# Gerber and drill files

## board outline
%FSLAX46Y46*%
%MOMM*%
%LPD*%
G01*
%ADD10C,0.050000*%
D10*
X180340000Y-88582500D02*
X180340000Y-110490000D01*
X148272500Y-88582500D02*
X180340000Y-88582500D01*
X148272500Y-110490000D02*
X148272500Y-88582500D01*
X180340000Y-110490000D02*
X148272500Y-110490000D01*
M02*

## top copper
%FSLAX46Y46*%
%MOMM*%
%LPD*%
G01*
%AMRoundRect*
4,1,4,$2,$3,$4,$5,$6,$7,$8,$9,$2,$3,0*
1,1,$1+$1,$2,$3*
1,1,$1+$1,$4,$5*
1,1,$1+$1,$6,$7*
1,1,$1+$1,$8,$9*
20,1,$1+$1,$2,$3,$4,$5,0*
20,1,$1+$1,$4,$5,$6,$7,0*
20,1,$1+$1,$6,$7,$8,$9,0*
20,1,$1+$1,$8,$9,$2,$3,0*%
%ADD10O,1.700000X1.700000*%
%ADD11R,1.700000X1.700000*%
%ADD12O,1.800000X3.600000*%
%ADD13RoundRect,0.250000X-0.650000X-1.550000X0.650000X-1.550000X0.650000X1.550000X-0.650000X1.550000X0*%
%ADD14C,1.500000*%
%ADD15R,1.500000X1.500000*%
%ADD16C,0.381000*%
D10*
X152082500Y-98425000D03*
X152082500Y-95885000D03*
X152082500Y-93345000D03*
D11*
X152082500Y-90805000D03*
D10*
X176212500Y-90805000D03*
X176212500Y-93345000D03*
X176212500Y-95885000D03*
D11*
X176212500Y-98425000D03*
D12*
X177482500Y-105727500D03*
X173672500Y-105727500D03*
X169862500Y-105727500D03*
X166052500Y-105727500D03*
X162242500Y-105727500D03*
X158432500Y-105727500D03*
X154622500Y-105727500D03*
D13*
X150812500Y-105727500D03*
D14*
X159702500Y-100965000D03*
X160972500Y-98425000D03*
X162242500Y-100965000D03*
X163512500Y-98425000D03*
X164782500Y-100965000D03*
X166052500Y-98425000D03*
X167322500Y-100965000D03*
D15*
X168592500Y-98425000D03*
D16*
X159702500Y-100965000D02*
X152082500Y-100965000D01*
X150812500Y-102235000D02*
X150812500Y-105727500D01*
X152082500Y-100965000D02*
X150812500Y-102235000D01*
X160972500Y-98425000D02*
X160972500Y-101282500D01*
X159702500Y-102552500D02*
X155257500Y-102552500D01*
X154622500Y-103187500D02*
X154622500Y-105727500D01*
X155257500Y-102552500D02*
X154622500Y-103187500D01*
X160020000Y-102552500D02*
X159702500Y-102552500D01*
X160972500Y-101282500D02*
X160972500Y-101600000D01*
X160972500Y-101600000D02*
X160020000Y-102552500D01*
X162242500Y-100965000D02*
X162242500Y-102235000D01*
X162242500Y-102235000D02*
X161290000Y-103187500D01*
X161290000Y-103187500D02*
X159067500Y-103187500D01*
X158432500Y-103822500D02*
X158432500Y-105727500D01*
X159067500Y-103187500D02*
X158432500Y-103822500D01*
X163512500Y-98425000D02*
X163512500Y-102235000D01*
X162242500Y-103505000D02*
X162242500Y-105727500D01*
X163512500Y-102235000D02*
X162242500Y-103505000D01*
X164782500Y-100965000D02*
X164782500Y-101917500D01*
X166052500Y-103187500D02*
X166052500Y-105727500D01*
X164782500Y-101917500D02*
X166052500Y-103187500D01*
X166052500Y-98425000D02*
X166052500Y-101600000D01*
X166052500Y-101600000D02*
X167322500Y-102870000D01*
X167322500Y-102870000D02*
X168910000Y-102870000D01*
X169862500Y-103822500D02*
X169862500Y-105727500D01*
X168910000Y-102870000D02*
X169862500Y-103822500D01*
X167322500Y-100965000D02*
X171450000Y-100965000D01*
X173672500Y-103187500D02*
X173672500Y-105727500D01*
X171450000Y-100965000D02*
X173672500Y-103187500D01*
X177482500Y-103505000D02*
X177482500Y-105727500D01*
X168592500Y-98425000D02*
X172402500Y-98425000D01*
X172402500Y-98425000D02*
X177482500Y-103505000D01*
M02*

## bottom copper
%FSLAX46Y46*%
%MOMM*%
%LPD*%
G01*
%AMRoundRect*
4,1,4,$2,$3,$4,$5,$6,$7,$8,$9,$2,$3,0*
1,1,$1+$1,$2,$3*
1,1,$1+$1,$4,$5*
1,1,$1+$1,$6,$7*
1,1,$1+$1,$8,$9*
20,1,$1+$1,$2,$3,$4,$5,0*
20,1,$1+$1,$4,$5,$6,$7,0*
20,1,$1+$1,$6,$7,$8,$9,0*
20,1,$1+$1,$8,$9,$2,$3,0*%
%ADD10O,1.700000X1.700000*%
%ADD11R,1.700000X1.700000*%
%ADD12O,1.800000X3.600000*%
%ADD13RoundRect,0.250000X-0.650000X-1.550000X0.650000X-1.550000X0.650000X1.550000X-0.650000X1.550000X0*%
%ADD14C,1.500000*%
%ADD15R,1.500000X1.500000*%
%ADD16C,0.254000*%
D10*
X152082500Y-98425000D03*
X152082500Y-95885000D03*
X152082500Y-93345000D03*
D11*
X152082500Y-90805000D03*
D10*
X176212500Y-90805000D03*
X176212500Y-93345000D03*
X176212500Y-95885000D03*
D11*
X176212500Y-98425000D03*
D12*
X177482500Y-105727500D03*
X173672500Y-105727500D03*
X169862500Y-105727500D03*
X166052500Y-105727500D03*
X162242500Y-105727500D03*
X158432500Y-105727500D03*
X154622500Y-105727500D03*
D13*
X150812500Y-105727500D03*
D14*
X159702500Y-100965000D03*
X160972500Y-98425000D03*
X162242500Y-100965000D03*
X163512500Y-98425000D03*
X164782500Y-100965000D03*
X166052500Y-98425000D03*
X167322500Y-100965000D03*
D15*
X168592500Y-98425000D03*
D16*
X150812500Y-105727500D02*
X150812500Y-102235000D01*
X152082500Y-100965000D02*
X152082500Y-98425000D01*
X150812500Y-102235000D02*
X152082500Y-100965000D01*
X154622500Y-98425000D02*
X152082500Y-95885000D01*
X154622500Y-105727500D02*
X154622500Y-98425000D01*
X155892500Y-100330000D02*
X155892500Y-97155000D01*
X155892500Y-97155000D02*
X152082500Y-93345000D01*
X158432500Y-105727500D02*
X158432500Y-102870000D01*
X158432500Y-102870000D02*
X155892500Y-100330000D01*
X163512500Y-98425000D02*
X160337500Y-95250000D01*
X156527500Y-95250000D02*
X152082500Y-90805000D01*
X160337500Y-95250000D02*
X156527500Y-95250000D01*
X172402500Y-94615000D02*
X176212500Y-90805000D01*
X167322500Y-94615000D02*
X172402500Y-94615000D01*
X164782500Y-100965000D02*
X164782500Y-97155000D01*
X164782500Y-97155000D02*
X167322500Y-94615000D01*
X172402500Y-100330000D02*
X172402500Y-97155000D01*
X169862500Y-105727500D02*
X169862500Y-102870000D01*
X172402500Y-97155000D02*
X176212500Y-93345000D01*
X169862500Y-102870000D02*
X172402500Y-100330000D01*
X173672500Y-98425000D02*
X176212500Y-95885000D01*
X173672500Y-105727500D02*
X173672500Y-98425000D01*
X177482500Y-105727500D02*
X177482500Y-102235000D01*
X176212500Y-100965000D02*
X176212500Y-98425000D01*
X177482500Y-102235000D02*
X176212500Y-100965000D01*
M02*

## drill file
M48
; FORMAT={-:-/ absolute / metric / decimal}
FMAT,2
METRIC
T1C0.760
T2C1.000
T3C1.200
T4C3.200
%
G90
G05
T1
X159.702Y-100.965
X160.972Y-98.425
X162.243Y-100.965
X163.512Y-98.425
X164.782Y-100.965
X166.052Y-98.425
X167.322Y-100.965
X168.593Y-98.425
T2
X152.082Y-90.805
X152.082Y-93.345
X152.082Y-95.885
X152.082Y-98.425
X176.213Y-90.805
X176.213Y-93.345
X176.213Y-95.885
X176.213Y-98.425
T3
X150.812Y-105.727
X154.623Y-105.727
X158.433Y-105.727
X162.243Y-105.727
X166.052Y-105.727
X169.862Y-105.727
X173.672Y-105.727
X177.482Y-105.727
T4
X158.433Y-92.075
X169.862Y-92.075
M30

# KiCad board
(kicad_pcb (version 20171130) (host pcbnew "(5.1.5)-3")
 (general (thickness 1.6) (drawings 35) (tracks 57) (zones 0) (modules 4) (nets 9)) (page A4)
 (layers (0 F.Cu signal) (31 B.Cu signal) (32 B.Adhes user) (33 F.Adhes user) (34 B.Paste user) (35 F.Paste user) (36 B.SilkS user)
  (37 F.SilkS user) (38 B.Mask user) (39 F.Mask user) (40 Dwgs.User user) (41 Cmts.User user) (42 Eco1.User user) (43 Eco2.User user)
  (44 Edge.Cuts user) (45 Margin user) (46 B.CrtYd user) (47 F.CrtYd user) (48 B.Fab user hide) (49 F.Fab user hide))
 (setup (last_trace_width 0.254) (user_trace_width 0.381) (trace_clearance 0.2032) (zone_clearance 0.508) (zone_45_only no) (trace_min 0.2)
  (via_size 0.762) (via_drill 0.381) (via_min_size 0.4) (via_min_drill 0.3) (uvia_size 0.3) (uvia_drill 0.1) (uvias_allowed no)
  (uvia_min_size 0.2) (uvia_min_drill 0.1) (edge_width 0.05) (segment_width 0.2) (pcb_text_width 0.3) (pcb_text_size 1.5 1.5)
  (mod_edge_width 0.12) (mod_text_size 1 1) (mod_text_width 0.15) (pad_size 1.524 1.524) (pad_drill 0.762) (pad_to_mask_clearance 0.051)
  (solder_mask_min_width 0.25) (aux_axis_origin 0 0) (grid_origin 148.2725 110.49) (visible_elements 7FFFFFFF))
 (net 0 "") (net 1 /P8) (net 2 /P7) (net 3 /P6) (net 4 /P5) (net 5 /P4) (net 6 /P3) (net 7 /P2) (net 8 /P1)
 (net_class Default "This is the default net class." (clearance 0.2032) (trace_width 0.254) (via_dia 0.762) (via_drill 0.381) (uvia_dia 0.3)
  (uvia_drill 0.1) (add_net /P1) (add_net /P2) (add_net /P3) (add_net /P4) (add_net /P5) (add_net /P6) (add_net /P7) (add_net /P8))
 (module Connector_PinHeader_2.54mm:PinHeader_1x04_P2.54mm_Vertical (layer F.Cu) (at 152.0825 90.805)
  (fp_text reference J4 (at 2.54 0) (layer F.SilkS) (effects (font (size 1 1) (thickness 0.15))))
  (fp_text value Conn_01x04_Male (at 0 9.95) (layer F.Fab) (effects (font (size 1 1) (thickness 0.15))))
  (pad 4 thru_hole oval (at 0 7.62) (size 1.7 1.7) (drill 1) (layers *.Cu *.Mask) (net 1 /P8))
  (pad 3 thru_hole oval (at 0 5.08) (size 1.7 1.7) (drill 1) (layers *.Cu *.Mask) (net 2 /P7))
  (pad 2 thru_hole oval (at 0 2.54) (size 1.7 1.7) (drill 1) (layers *.Cu *.Mask) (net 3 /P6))
  (pad 1 thru_hole rect (at 0 0) (size 1.7 1.7) (drill 1) (layers *.Cu *.Mask) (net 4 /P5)))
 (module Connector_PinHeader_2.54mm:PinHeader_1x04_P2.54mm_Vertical (layer F.Cu) (at 176.2125 98.425 180)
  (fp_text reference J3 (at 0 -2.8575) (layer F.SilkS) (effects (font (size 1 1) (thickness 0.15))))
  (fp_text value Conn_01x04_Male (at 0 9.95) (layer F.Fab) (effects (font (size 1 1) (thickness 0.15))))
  (pad 4 thru_hole oval (at 0 7.62 180) (size 1.7 1.7) (drill 1) (layers *.Cu *.Mask) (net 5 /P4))
  (pad 3 thru_hole oval (at 0 5.08 180) (size 1.7 1.7) (drill 1) (layers *.Cu *.Mask) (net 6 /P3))
  (pad 2 thru_hole oval (at 0 2.54 180) (size 1.7 1.7) (drill 1) (layers *.Cu *.Mask) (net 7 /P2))
  (pad 1 thru_hole rect (at 0 0 180) (size 1.7 1.7) (drill 1) (layers *.Cu *.Mask) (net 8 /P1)))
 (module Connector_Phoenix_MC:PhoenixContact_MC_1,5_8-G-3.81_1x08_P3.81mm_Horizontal (layer F.Cu) (at 150.8125 105.7275)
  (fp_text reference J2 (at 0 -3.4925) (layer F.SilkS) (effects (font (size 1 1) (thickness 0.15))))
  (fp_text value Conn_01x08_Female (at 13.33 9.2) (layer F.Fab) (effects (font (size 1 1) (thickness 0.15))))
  (pad 8 thru_hole oval (at 26.67 0) (size 1.8 3.6) (drill 1.2) (layers *.Cu *.Mask) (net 8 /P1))
  (pad 7 thru_hole oval (at 22.86 0) (size 1.8 3.6) (drill 1.2) (layers *.Cu *.Mask) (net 7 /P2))
  (pad 6 thru_hole oval (at 19.05 0) (size 1.8 3.6) (drill 1.2) (layers *.Cu *.Mask) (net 6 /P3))
  (pad 5 thru_hole oval (at 15.24 0) (size 1.8 3.6) (drill 1.2) (layers *.Cu *.Mask) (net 5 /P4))
  (pad 4 thru_hole oval (at 11.43 0) (size 1.8 3.6) (drill 1.2) (layers *.Cu *.Mask) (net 4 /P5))
  (pad 3 thru_hole oval (at 7.62 0) (size 1.8 3.6) (drill 1.2) (layers *.Cu *.Mask) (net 3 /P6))
  (pad 2 thru_hole oval (at 3.81 0) (size 1.8 3.6) (drill 1.2) (layers *.Cu *.Mask) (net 2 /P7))
  (pad 1 thru_hole roundrect (at 0 0) (size 1.8 3.6) (drill 1.2) (layers *.Cu *.Mask) (roundrect_rratio 0.138889) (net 1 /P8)))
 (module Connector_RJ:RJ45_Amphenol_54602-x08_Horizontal (layer F.Cu) (at 168.5925 98.425 180)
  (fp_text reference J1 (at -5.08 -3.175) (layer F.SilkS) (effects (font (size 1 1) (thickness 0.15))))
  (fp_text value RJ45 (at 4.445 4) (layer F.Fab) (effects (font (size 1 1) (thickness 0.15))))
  (pad 8 thru_hole circle (at 8.89 -2.54 180) (size 1.5 1.5) (drill 0.76) (layers *.Cu *.Mask) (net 1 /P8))
  (pad 7 thru_hole circle (at 7.62 0 180) (size 1.5 1.5) (drill 0.76) (layers *.Cu *.Mask) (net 2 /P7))
  (pad 6 thru_hole circle (at 6.35 -2.54 180) (size 1.5 1.5) (drill 0.76) (layers *.Cu *.Mask) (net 3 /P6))
  (pad 5 thru_hole circle (at 5.08 0 180) (size 1.5 1.5) (drill 0.76) (layers *.Cu *.Mask) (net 4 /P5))
  (pad 4 thru_hole circle (at 3.81 -2.54 180) (size 1.5 1.5) (drill 0.76) (layers *.Cu *.Mask) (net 5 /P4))
  (pad 3 thru_hole circle (at 2.54 0 180) (size 1.5 1.5) (drill 0.76) (layers *.Cu *.Mask) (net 6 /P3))
  (pad 2 thru_hole circle (at 1.27 -2.54 180) (size 1.5 1.5) (drill 0.76) (layers *.Cu *.Mask) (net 7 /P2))
  (pad 1 thru_hole rect (at 0 0 180) (size 1.5 1.5) (drill 0.76) (layers *.Cu *.Mask) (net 8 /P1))
  (pad "" np_thru_hole circle (at -1.27 6.35 180) (size 3.2 3.2) (drill 3.2) (layers *.Cu *.Mask))
  (pad "" np_thru_hole circle (at 10.16 6.35 180) (size 3.2 3.2) (drill 3.2) (layers *.Cu *.Mask)))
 (gr_line (start 180.34 88.5825) (end 180.34 110.49) (layer Edge.Cuts) (width 0.05))
 (gr_line (start 148.2725 88.5825) (end 180.34 88.5825) (layer Edge.Cuts) (width 0.05))
 (gr_line (start 148.2725 110.49) (end 148.2725 88.5825) (layer Edge.Cuts) (width 0.05))
 (gr_line (start 180.34 110.49) (end 148.2725 110.49) (layer Edge.Cuts) (width 0.05))
 (segment (start 159.7025 100.965) (end 152.0825 100.965) (width 0.381) (layer F.Cu) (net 1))
 (segment (start 150.8125 102.235) (end 150.8125 105.7275) (width 0.381) (layer F.Cu) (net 1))
 (segment (start 152.0825 100.965) (end 150.8125 102.235) (width 0.381) (layer F.Cu) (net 1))
 (segment (start 150.8125 105.7275) (end 150.8125 102.235) (width 0.254) (layer B.Cu) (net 1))
 (segment (start 152.0825 100.965) (end 152.0825 98.425) (width 0.254) (layer B.Cu) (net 1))
 (segment (start 150.8125 102.235) (end 152.0825 100.965) (width 0.254) (layer B.Cu) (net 1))
 (segment (start 160.9725 98.425) (end 160.9725 101.2825) (width 0.381) (layer F.Cu) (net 2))
 (segment (start 159.7025 102.5525) (end 155.2575 102.5525) (width 0.381) (layer F.Cu) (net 2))
 (segment (start 154.6225 103.1875) (end 154.6225 105.7275) (width 0.381) (layer F.Cu) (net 2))
 (segment (start 155.2575 102.5525) (end 154.6225 103.1875) (width 0.381) (layer F.Cu) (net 2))
 (segment (start 160.02 102.5525) (end 159.7025 102.5525) (width 0.381) (layer F.Cu) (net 2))
 (segment (start 160.9725 101.2825) (end 160.9725 101.6) (width 0.381) (layer F.Cu) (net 2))
 (segment (start 160.9725 101.6) (end 160.02 102.5525) (width 0.381) (layer F.Cu) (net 2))
 (segment (start 154.6225 98.425) (end 152.0825 95.885) (width 0.254) (layer B.Cu) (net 2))
 (segment (start 154.6225 105.7275) (end 154.6225 98.425) (width 0.254) (layer B.Cu) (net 2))
 (segment (start 162.2425 100.965) (end 162.2425 102.235) (width 0.381) (layer F.Cu) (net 3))
 (segment (start 162.2425 102.235) (end 161.29 103.1875) (width 0.381) (layer F.Cu) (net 3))
 (segment (start 161.29 103.1875) (end 159.0675 103.1875) (width 0.381) (layer F.Cu) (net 3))
 (segment (start 158.4325 103.8225) (end 158.4325 105.7275) (width 0.381) (layer F.Cu) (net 3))
 (segment (start 159.0675 103.1875) (end 158.4325 103.8225) (width 0.381) (layer F.Cu) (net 3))
 (segment (start 155.8925 100.33) (end 155.8925 97.155) (width 0.254) (layer B.Cu) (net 3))
 (segment (start 155.8925 97.155) (end 152.0825 93.345) (width 0.254) (layer B.Cu) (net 3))
 (segment (start 158.4325 105.7275) (end 158.4325 102.87) (width 0.254) (layer B.Cu) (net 3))
 (segment (start 158.4325 102.87) (end 155.8925 100.33) (width 0.254) (layer B.Cu) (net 3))
 (segment (start 163.5125 98.425) (end 163.5125 102.235) (width 0.381) (layer F.Cu) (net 4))
 (segment (start 162.2425 103.505) (end 162.2425 105.7275) (width 0.381) (layer F.Cu) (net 4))
 (segment (start 163.5125 102.235) (end 162.2425 103.505) (width 0.381) (layer F.Cu) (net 4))
 (segment (start 163.5125 98.425) (end 160.3375 95.25) (width 0.254) (layer B.Cu) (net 4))
 (segment (start 156.5275 95.25) (end 152.0825 90.805) (width 0.254) (layer B.Cu) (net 4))
 (segment (start 160.3375 95.25) (end 156.5275 95.25) (width 0.254) (layer B.Cu) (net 4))
 (segment (start 164.7825 100.965) (end 164.7825 101.9175) (width 0.381) (layer F.Cu) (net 5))
 (segment (start 166.0525 103.1875) (end 166.0525 105.7275) (width 0.381) (layer F.Cu) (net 5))
 (segment (start 164.7825 101.9175) (end 166.0525 103.1875) (width 0.381) (layer F.Cu) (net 5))
 (segment (start 172.4025 94.615) (end 176.2125 90.805) (width 0.254) (layer B.Cu) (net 5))
 (segment (start 167.3225 94.615) (end 172.4025 94.615) (width 0.254) (layer B.Cu) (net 5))
 (segment (start 164.7825 100.965) (end 164.7825 97.155) (width 0.254) (layer B.Cu) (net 5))
 (segment (start 164.7825 97.155) (end 167.3225 94.615) (width 0.254) (layer B.Cu) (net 5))
 (segment (start 166.0525 98.425) (end 166.0525 101.6) (width 0.381) (layer F.Cu) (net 6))
 (segment (start 166.0525 101.6) (end 167.3225 102.87) (width 0.381) (layer F.Cu) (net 6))
 (segment (start 167.3225 102.87) (end 168.91 102.87) (width 0.381) (layer F.Cu) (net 6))
 (segment (start 169.8625 103.8225) (end 169.8625 105.7275) (width 0.381) (layer F.Cu) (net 6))
 (segment (start 168.91 102.87) (end 169.8625 103.8225) (width 0.381) (layer F.Cu) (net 6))
 (segment (start 172.4025 100.33) (end 172.4025 97.155) (width 0.254) (layer B.Cu) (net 6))
 (segment (start 169.8625 105.7275) (end 169.8625 102.87) (width 0.254) (layer B.Cu) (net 6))
 (segment (start 172.4025 97.155) (end 176.2125 93.345) (width 0.254) (layer B.Cu) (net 6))
 (segment (start 169.8625 102.87) (end 172.4025 100.33) (width 0.254) (layer B.Cu) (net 6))
 (segment (start 167.3225 100.965) (end 171.45 100.965) (width 0.381) (layer F.Cu) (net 7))
 (segment (start 173.6725 103.1875) (end 173.6725 105.7275) (width 0.381) (layer F.Cu) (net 7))
 (segment (start 171.45 100.965) (end 173.6725 103.1875) (width 0.381) (layer F.Cu) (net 7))
 (segment (start 173.6725 98.425) (end 176.2125 95.885) (width 0.254) (layer B.Cu) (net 7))
 (segment (start 173.6725 105.7275) (end 173.6725 98.425) (width 0.254) (layer B.Cu) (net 7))
 (segment (start 177.4825 103.505) (end 177.4825 105.7275) (width 0.381) (layer F.Cu) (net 8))
 (segment (start 168.5925 98.425) (end 172.4025 98.425) (width 0.381) (layer F.Cu) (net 8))
 (segment (start 172.4025 98.425) (end 177.4825 103.505) (width 0.381) (layer F.Cu) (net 8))
 (segment (start 177.4825 105.7275) (end 177.4825 102.235) (width 0.254) (layer B.Cu) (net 8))
 (segment (start 176.2125 100.965) (end 176.2125 98.425) (width 0.254) (layer B.Cu) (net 8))
 (segment (start 177.4825 102.235) (end 176.2125 100.965) (width 0.254) (layer B.Cu) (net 8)))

